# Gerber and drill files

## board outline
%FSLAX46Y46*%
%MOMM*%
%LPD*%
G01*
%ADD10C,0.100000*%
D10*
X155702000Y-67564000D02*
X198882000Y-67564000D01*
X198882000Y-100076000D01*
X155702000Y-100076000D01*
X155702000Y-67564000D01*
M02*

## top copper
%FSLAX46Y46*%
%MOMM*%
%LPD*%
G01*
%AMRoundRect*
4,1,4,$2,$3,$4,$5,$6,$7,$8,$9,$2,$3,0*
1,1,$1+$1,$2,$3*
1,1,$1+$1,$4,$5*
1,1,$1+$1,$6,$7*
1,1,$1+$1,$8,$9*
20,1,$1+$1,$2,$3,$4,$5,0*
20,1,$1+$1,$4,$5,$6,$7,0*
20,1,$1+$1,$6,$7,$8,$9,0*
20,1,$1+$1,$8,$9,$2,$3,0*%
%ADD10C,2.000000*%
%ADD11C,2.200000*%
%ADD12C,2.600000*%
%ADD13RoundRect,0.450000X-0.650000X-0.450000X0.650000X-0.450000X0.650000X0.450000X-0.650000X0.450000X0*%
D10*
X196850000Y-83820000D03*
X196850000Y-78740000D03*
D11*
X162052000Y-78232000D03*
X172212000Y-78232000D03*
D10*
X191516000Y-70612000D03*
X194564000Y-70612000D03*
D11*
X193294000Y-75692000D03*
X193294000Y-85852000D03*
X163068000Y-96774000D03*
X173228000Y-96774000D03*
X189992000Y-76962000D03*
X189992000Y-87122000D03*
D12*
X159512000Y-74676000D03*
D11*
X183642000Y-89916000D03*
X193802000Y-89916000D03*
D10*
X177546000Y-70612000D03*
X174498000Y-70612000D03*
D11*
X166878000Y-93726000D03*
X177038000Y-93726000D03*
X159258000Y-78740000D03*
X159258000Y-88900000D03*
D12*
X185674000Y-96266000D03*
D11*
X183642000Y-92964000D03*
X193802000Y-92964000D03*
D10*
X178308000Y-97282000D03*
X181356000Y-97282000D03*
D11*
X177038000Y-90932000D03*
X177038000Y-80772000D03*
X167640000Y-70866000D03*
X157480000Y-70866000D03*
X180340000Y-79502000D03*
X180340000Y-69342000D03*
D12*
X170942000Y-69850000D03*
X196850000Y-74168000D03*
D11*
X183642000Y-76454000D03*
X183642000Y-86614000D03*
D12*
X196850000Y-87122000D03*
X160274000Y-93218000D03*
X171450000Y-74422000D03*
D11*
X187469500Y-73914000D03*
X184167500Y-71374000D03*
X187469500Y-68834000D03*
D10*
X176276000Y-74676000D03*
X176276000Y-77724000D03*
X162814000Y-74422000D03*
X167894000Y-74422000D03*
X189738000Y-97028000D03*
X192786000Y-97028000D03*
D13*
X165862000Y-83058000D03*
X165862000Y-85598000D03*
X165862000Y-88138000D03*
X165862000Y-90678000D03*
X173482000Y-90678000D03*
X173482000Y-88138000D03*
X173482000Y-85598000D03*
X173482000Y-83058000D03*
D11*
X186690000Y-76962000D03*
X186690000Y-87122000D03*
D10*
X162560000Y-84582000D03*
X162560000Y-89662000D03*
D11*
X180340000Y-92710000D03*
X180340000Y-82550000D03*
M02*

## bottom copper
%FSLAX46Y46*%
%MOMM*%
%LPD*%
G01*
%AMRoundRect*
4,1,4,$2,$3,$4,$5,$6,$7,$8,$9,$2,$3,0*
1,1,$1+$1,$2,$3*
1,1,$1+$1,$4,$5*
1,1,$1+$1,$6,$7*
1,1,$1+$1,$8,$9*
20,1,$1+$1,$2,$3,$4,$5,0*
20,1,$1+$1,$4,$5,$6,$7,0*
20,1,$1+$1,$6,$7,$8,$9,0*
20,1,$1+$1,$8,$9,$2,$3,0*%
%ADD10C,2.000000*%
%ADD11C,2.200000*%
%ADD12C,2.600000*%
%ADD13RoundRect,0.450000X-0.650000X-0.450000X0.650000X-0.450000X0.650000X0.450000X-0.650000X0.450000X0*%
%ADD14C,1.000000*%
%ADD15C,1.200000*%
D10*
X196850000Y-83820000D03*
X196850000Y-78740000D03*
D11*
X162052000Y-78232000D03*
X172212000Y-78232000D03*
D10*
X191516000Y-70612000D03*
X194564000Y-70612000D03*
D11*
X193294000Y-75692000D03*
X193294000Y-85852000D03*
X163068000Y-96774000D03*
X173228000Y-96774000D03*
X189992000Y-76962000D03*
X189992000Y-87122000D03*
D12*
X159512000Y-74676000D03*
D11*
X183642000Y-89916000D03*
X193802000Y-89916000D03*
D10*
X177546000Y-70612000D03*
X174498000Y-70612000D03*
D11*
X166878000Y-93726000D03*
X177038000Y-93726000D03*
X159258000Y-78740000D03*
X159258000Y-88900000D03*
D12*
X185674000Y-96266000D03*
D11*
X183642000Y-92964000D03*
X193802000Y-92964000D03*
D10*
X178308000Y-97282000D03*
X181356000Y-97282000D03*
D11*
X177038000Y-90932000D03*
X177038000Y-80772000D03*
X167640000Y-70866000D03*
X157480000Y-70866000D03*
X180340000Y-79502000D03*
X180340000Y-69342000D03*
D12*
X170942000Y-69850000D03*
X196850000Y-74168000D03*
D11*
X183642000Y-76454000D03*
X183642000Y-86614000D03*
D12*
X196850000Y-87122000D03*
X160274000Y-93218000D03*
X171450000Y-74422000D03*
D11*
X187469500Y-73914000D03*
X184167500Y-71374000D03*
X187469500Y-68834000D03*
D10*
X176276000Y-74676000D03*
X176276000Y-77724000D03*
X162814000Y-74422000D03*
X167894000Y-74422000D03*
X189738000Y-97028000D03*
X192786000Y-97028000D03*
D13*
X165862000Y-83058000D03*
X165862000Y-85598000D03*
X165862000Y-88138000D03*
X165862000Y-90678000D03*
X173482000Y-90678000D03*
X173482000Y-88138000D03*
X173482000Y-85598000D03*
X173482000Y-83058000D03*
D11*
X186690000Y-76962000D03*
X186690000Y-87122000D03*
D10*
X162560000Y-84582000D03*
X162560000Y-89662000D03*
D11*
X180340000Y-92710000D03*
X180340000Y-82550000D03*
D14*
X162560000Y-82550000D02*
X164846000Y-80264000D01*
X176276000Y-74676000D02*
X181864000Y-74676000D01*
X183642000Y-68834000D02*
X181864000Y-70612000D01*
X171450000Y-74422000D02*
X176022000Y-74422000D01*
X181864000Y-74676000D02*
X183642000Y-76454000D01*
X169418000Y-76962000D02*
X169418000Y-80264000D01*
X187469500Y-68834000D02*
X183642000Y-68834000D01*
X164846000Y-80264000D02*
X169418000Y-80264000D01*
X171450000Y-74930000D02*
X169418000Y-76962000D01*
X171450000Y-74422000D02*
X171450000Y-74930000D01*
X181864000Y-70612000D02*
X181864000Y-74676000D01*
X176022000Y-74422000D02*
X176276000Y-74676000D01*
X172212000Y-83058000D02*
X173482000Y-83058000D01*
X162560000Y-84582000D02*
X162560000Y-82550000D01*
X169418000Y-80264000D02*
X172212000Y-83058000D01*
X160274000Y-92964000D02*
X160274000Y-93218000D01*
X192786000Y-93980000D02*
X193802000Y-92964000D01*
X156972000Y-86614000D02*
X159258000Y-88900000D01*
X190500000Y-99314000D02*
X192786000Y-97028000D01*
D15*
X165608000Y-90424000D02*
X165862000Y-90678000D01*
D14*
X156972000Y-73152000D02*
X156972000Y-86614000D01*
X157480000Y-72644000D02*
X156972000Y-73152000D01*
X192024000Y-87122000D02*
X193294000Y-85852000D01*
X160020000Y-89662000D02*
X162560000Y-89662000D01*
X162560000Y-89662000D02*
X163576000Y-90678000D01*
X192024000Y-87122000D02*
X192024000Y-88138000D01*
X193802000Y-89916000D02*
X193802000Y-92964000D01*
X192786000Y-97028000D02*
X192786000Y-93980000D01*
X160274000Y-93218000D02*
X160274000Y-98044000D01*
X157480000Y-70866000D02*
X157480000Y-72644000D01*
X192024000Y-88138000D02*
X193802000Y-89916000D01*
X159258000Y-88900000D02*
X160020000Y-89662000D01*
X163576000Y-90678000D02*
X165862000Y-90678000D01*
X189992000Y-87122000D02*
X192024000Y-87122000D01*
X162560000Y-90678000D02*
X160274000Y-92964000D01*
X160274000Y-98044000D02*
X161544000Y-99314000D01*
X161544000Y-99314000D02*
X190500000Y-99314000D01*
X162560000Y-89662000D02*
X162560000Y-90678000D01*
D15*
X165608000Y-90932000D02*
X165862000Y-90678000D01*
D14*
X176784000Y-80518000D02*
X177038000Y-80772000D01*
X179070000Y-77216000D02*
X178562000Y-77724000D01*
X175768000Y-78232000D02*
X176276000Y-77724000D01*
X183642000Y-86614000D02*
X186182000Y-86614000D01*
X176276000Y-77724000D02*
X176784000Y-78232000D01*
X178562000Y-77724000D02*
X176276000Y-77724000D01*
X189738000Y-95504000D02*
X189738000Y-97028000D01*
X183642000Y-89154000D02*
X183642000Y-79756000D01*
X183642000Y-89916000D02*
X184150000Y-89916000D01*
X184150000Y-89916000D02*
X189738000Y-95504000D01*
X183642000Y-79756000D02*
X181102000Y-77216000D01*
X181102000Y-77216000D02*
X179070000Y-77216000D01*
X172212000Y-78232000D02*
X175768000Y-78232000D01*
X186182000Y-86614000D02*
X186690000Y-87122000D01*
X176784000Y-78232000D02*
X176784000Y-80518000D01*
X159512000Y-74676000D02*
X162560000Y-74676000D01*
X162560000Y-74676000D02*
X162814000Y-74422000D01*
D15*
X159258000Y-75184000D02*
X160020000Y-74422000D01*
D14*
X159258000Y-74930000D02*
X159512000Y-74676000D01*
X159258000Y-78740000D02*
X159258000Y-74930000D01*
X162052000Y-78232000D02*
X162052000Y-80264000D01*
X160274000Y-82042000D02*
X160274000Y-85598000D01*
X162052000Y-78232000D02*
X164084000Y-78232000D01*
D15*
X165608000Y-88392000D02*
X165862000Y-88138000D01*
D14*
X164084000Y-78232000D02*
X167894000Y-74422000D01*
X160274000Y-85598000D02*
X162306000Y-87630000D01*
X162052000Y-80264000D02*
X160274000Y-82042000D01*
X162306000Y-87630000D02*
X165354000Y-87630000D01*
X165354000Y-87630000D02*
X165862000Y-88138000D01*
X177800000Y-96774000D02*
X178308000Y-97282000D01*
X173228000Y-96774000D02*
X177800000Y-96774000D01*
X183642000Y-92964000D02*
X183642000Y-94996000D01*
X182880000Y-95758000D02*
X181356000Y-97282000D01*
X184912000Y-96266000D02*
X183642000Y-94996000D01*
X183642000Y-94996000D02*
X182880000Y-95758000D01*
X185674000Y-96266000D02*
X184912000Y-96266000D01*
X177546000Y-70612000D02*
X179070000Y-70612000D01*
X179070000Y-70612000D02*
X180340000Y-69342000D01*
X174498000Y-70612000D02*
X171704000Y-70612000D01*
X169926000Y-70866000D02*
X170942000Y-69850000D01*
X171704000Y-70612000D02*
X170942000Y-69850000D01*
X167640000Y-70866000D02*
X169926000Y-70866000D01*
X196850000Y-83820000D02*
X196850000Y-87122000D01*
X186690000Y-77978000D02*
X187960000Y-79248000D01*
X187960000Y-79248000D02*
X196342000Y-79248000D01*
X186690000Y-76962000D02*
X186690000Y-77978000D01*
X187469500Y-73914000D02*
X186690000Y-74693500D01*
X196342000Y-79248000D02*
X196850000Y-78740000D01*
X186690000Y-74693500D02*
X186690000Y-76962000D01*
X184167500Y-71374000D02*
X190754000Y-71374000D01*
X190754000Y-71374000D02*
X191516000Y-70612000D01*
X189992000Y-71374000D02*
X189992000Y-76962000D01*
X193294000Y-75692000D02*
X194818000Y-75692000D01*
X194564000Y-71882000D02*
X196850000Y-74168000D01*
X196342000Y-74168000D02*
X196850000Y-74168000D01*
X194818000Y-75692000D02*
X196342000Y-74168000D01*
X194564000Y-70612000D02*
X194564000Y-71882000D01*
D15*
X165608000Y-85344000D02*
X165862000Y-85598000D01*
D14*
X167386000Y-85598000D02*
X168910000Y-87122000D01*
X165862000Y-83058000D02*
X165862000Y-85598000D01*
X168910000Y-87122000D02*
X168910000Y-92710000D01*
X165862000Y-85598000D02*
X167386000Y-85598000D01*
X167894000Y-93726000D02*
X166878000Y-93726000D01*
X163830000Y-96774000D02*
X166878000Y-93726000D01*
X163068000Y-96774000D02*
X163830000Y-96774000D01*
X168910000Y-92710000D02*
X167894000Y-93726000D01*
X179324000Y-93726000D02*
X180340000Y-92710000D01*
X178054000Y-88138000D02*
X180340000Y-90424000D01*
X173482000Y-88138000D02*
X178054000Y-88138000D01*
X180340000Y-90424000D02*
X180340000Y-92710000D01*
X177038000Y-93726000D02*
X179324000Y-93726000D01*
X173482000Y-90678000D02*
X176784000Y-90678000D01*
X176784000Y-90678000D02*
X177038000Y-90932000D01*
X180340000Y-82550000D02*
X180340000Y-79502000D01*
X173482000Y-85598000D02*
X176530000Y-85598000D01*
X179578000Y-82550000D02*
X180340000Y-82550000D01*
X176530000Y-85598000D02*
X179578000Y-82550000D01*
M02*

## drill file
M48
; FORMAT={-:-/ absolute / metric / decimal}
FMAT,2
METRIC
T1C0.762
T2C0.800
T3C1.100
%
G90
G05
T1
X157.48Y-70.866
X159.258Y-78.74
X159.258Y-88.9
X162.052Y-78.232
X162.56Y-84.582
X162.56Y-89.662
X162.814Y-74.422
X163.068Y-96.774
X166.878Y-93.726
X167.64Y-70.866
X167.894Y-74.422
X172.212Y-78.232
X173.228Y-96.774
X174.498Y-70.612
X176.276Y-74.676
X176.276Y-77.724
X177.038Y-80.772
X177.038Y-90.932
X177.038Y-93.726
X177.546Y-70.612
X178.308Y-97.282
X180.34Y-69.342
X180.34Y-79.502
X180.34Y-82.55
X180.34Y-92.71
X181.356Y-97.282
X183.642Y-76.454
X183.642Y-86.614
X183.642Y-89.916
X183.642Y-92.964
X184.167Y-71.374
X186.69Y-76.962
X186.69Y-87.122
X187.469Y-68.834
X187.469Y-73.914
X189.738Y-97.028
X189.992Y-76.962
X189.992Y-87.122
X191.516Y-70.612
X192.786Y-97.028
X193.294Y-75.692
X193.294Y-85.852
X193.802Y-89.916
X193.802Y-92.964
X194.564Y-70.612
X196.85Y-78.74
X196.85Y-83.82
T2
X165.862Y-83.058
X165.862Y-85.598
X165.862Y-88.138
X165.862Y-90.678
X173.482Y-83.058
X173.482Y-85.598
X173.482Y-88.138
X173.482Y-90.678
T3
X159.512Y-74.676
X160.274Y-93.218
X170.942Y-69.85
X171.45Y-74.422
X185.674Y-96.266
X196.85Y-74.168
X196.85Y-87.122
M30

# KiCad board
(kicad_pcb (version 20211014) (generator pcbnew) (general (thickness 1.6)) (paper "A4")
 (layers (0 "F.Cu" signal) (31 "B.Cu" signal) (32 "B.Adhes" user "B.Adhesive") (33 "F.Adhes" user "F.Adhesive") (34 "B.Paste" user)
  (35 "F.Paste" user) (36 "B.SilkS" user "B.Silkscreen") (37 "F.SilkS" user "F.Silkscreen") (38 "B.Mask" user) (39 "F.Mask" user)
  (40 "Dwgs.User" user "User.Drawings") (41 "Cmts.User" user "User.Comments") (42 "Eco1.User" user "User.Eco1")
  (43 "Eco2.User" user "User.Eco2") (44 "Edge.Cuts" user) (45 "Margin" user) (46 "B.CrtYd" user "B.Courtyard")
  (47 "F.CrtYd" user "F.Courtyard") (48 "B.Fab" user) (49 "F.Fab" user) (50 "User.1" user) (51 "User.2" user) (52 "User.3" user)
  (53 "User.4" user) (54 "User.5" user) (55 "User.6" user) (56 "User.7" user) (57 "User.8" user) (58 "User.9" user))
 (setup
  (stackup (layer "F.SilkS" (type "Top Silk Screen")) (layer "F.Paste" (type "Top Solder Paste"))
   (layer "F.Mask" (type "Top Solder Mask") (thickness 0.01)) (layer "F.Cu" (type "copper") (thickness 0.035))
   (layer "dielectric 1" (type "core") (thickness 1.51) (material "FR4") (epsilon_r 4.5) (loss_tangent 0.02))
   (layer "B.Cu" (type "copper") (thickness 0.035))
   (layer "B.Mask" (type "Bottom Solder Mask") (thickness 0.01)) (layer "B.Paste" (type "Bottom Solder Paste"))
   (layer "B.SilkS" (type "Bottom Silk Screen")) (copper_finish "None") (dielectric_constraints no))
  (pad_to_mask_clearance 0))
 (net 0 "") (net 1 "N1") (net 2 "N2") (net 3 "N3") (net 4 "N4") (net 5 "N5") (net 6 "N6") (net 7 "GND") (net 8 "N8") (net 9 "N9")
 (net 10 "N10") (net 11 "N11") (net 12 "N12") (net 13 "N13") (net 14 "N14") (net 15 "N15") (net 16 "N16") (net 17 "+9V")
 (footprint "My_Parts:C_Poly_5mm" (layer "F.Cu") (at 196.85 81.28 90)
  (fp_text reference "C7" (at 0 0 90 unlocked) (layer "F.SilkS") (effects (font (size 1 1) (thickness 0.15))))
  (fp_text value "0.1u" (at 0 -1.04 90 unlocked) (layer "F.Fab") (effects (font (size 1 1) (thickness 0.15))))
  (pad "1" thru_hole circle (at -2.54 0 90) (size 2 2) (drill 0.762) (layers *.Cu *.Mask) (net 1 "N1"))
  (pad "2" thru_hole circle (at 2.54 0 90) (size 2 2) (drill 0.762) (layers *.Cu *.Mask) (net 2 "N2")))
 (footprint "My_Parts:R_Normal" (layer "F.Cu") (at 167.132 78.232)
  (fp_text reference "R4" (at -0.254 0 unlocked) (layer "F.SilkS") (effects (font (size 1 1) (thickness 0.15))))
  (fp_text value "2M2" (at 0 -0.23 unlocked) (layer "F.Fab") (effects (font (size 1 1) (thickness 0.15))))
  (pad "1" thru_hole circle (at -5.08 0) (size 2.2 2.2) (drill 0.762) (layers *.Cu *.Mask) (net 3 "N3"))
  (pad "2" thru_hole circle (at 5.08 0) (size 2.2 2.2) (drill 0.762) (layers *.Cu *.Mask) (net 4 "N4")))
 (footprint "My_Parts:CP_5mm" (layer "F.Cu") (at 193.04 70.612)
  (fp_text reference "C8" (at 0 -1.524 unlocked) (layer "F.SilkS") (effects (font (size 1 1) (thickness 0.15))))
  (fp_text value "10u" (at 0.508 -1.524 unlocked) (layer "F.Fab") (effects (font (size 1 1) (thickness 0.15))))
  (pad "1" thru_hole circle (at -1.524 0) (size 2 2) (drill 0.762) (layers *.Cu *.Mask) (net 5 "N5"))
  (pad "2" thru_hole circle (at 1.524 0) (size 2 2) (drill 0.762) (layers *.Cu *.Mask) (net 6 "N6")))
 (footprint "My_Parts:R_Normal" (layer "F.Cu") (at 193.294 80.772 -90)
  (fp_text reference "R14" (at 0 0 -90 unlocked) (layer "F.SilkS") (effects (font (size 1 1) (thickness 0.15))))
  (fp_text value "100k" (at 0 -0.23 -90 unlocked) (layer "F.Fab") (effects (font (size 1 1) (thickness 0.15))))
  (pad "1" thru_hole circle (at -5.08 0 270) (size 2.2 2.2) (drill 0.762) (layers *.Cu *.Mask) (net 6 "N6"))
  (pad "2" thru_hole circle (at 5.08 0 270) (size 2.2 2.2) (drill 0.762) (layers *.Cu *.Mask) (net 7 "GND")))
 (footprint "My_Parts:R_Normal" (layer "F.Cu") (at 168.148 96.774)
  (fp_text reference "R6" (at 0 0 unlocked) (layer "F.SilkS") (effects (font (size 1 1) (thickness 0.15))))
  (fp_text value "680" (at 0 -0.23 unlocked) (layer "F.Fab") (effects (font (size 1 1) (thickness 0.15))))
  (pad "1" thru_hole circle (at -5.08 0) (size 2.2 2.2) (drill 0.762) (layers *.Cu *.Mask) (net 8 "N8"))
  (pad "2" thru_hole circle (at 5.08 0) (size 2.2 2.2) (drill 0.762) (layers *.Cu *.Mask) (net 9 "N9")))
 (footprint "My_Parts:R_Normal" (layer "F.Cu") (at 189.992 82.042 -90)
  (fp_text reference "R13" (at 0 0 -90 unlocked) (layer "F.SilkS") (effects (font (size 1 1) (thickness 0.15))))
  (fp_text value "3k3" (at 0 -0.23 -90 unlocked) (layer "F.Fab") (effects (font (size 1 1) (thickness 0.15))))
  (pad "1" thru_hole circle (at -5.08 0 270) (size 2.2 2.2) (drill 0.762) (layers *.Cu *.Mask) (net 5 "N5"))
  (pad "2" thru_hole circle (at 5.08 0 270) (size 2.2 2.2) (drill 0.762) (layers *.Cu *.Mask) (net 7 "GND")))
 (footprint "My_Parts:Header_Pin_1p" (layer "F.Cu") (at 159.512 74.676)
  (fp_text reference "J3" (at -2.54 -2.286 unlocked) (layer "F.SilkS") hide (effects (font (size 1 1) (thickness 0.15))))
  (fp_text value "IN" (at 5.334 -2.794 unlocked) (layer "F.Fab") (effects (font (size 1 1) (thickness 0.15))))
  (pad "1" thru_hole circle (at 0 0) (size 2.6 2.6) (drill 1.1) (layers *.Cu *.Mask) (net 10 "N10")))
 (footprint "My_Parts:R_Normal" (layer "F.Cu") (at 188.722 89.916)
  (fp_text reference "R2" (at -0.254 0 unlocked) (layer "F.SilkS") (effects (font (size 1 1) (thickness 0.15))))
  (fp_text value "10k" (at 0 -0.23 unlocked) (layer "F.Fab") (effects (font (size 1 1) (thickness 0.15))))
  (pad "1" thru_hole circle (at -5.08 0) (size 2.2 2.2) (drill 0.762) (layers *.Cu *.Mask) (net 4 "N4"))
  (pad "2" thru_hole circle (at 5.08 0) (size 2.2 2.2) (drill 0.762) (layers *.Cu *.Mask) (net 7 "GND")))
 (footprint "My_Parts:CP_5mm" (layer "F.Cu") (at 176.022 70.612 180)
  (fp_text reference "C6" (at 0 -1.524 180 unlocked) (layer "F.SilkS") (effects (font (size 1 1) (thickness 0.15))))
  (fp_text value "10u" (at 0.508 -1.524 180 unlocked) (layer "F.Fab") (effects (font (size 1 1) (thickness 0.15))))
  (pad "1" thru_hole circle (at -1.524 0 180) (size 2 2) (drill 0.762) (layers *.Cu *.Mask) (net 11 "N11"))
  (pad "2" thru_hole circle (at 1.524 0 180) (size 2 2) (drill 0.762) (layers *.Cu *.Mask) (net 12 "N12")))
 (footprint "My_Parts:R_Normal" (layer "F.Cu") (at 171.958 93.726)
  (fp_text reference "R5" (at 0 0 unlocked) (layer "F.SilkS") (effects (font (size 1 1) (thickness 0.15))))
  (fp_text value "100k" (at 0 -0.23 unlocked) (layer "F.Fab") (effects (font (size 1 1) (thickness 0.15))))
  (pad "1" thru_hole circle (at -5.08 0) (size 2.2 2.2) (drill 0.762) (layers *.Cu *.Mask) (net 8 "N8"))
  (pad "2" thru_hole circle (at 5.08 0) (size 2.2 2.2) (drill 0.762) (layers *.Cu *.Mask) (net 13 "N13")))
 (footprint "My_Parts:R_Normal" (layer "F.Cu") (at 159.258 83.82 -90)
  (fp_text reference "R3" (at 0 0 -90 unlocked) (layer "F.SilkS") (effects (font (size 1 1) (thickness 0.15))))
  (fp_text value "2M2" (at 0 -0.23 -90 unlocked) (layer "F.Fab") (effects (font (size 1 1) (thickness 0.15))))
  (pad "1" thru_hole circle (at -5.08 0 270) (size 2.2 2.2) (drill 0.762) (layers *.Cu *.Mask) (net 10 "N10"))
  (pad "2" thru_hole circle (at 5.08 0 270) (size 2.2 2.2) (drill 0.762) (layers *.Cu *.Mask) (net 7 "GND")))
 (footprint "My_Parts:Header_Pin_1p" (layer "F.Cu") (at 185.674 96.266)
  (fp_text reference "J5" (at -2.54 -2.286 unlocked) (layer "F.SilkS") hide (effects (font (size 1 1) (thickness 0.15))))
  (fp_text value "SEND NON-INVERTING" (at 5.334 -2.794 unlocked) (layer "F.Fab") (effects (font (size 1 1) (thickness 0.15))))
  (pad "1" thru_hole circle (at 0 0) (size 2.6 2.6) (drill 1.1) (layers *.Cu *.Mask) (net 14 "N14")))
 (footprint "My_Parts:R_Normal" (layer "F.Cu") (at 188.722 92.964)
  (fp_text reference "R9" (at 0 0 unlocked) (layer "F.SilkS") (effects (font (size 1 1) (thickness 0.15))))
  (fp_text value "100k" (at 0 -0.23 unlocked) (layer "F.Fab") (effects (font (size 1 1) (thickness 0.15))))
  (pad "1" thru_hole circle (at -5.08 0) (size 2.2 2.2) (drill 0.762) (layers *.Cu *.Mask) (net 14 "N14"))
  (pad "2" thru_hole circle (at 5.08 0) (size 2.2 2.2) (drill 0.762) (layers *.Cu *.Mask) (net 7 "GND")))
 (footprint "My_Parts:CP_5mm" (layer "F.Cu") (at 179.832 97.282)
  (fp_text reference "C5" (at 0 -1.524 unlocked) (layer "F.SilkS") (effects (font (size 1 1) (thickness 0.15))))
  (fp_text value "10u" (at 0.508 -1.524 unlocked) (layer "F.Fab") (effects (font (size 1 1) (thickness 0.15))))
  (pad "1" thru_hole circle (at -1.524 0) (size 2 2) (drill 0.762) (layers *.Cu *.Mask) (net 9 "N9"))
  (pad "2" thru_hole circle (at 1.524 0) (size 2 2) (drill 0.762) (layers *.Cu *.Mask) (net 14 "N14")))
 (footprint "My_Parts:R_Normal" (layer "F.Cu") (at 177.038 85.852 90)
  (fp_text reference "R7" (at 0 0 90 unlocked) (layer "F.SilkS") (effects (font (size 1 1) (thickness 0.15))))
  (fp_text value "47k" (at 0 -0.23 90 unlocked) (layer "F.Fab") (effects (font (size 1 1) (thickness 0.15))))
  (pad "1" thru_hole circle (at -5.08 0 90) (size 2.2 2.2) (drill 0.762) (layers *.Cu *.Mask) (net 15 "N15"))
  (pad "2" thru_hole circle (at 5.08 0 90) (size 2.2 2.2) (drill 0.762) (layers *.Cu *.Mask) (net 4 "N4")))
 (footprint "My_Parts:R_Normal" (layer "F.Cu") (at 162.56 70.866 180)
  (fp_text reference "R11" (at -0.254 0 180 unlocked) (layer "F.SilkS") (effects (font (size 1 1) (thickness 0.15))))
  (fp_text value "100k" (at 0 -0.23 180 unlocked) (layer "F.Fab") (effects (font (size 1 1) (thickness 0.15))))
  (pad "1" thru_hole circle (at -5.08 0 180) (size 2.2 2.2) (drill 0.762) (layers *.Cu *.Mask) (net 12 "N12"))
  (pad "2" thru_hole circle (at 5.08 0 180) (size 2.2 2.2) (drill 0.762) (layers *.Cu *.Mask) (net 7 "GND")))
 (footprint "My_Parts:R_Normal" (layer "F.Cu") (at 180.34 74.422 90)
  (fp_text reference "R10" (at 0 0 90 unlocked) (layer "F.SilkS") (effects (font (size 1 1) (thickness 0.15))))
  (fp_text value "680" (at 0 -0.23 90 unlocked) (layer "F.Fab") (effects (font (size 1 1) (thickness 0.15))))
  (pad "1" thru_hole circle (at -5.08 0 90) (size 2.2 2.2) (drill 0.762) (layers *.Cu *.Mask) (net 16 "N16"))
  (pad "2" thru_hole circle (at 5.08 0 90) (size 2.2 2.2) (drill 0.762) (layers *.Cu *.Mask) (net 11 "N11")))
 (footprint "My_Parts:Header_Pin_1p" (layer "F.Cu") (at 170.942 69.85)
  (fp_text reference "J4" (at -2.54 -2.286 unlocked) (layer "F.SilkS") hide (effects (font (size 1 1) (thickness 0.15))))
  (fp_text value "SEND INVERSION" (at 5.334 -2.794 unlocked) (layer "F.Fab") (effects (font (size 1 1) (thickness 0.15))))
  (pad "1" thru_hole circle (at 0 0) (size 2.6 2.6) (drill 1.1) (layers *.Cu *.Mask) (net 12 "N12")))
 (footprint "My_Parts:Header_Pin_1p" (layer "F.Cu") (at 196.85 74.168)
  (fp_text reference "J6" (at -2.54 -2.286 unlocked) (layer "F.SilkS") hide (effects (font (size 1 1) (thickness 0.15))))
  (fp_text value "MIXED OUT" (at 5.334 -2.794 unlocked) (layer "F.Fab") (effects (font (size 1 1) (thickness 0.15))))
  (pad "1" thru_hole circle (at 0 0) (size 2.6 2.6) (drill 1.1) (layers *.Cu *.Mask) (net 6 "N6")))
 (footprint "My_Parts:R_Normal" (layer "F.Cu") (at 183.642 81.534 -90)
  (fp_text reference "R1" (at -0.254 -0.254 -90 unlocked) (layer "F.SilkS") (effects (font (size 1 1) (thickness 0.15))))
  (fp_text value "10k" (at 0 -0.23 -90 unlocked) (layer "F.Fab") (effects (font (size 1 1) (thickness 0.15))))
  (pad "1" thru_hole circle (at -5.08 0 270) (size 2.2 2.2) (drill 0.762) (layers *.Cu *.Mask) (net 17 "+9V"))
  (pad "2" thru_hole circle (at 5.08 0 270) (size 2.2 2.2) (drill 0.762) (layers *.Cu *.Mask) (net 4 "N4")))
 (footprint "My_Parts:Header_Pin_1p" (layer "F.Cu") (at 196.85 87.122)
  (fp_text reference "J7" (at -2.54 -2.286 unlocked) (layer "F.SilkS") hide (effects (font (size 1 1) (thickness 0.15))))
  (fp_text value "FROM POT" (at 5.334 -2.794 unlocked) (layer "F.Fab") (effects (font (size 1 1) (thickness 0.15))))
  (pad "1" thru_hole circle (at 0 0) (size 2.6 2.6) (drill 1.1) (layers *.Cu *.Mask) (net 1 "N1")))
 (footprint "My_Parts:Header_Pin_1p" (layer "F.Cu") (at 160.274 93.218)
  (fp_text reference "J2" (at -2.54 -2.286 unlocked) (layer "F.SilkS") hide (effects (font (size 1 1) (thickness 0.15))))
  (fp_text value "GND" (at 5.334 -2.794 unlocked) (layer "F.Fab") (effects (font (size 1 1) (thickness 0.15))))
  (pad "1" thru_hole circle (at 0 0) (size 2.6 2.6) (drill 1.1) (layers *.Cu *.Mask) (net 7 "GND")))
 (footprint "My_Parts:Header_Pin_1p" (layer "F.Cu") (at 171.45 74.422)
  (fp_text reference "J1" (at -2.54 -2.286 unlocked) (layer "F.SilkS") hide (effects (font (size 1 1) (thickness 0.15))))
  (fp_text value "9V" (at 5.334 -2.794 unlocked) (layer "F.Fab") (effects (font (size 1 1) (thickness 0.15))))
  (pad "1" thru_hole circle (at 0 0) (size 2.6 2.6) (drill 1.1) (layers *.Cu *.Mask) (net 17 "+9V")))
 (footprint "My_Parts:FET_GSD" (layer "F.Cu") (at 186.4535 73.914 90)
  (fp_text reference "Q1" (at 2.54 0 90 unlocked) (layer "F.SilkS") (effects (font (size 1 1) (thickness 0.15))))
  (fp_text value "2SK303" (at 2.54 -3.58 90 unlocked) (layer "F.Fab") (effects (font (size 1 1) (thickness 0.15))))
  (pad "1" thru_hole circle (at 0 1.016 90) (size 2.2 2.2) (drill 0.762) (layers *.Cu *.Mask) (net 2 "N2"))
  (pad "2" thru_hole circle (at 2.54 -2.286 90) (size 2.2 2.2) (drill 0.762) (layers *.Cu *.Mask) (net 5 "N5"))
  (pad "3" thru_hole circle (at 5.08 1.016 90) (size 2.2 2.2) (drill 0.762) (layers *.Cu *.Mask) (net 17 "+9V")))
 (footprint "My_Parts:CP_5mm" (layer "F.Cu") (at 176.276 76.2 -90)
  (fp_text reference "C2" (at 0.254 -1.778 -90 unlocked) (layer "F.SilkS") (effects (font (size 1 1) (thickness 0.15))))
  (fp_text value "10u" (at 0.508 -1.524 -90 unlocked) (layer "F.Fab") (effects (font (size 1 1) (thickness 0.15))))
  (pad "1" thru_hole circle (at -1.524 0 270) (size 2 2) (drill 0.762) (layers *.Cu *.Mask) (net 17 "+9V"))
  (pad "2" thru_hole circle (at 1.524 0 270) (size 2 2) (drill 0.762) (layers *.Cu *.Mask) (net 4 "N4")))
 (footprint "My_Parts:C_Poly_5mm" (layer "F.Cu") (at 165.354 74.422)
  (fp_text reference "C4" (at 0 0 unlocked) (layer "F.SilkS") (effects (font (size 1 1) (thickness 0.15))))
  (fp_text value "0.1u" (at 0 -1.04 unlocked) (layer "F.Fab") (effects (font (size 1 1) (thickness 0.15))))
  (pad "1" thru_hole circle (at -2.54 0) (size 2 2) (drill 0.762) (layers *.Cu *.Mask) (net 10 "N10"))
  (pad "2" thru_hole circle (at 2.54 0) (size 2 2) (drill 0.762) (layers *.Cu *.Mask) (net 3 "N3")))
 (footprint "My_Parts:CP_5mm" (layer "F.Cu") (at 191.262 97.028)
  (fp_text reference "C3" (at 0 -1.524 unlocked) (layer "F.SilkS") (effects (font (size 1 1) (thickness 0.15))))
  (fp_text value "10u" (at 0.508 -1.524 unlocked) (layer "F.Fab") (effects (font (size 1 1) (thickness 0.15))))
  (pad "1" thru_hole circle (at -1.524 0) (size 2 2) (drill 0.762) (layers *.Cu *.Mask) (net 4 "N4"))
  (pad "2" thru_hole circle (at 1.524 0) (size 2 2) (drill 0.762) (layers *.Cu *.Mask) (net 7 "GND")))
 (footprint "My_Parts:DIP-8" (layer "F.Cu") (at 167.132 83.558)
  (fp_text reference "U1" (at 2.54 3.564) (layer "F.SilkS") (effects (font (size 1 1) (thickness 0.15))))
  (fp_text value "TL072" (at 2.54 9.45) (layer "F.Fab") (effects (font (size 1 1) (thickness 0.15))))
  (pad "1" thru_hole roundrect (at -1.27 -0.5) (size 2.2 1.8) (drill 0.8) (layers *.Cu *.Mask) (roundrect_rratio 0.25) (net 8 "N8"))
  (pad "2" thru_hole roundrect (at -1.27 2.04) (size 2.2 1.8) (drill 0.8) (layers *.Cu *.Mask) (roundrect_rratio 0.25) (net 8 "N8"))
  (pad "3" thru_hole roundrect (at -1.27 4.58) (size 2.2 1.8) (drill 0.8) (layers *.Cu *.Mask) (roundrect_rratio 0.25) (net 3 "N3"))
  (pad "4" thru_hole roundrect (at -1.27 7.12) (size 2.2 1.8) (drill 0.8) (layers *.Cu *.Mask) (roundrect_rratio 0.25) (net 7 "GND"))
  (pad "5" thru_hole roundrect (at 6.35 7.12) (size 2.2 1.8) (drill 0.8) (layers *.Cu *.Mask) (roundrect_rratio 0.25) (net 15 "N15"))
  (pad "6" thru_hole roundrect (at 6.35 4.58) (size 2.2 1.8) (drill 0.8) (layers *.Cu *.Mask) (roundrect_rratio 0.25) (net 13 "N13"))
  (pad "7" thru_hole roundrect (at 6.35 2.04) (size 2.2 1.8) (drill 0.8) (layers *.Cu *.Mask) (roundrect_rratio 0.25) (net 16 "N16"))
  (pad "8" thru_hole roundrect (at 6.35 -0.5) (size 2.2 1.8) (drill 0.8) (layers *.Cu *.Mask) (roundrect_rratio 0.25) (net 17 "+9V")))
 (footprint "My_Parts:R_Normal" (layer "F.Cu") (at 186.69 82.042 -90)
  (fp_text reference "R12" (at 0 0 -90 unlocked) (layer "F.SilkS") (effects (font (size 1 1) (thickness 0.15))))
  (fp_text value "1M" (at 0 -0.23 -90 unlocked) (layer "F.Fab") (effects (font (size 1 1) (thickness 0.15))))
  (pad "1" thru_hole circle (at -5.08 0 270) (size 2.2 2.2) (drill 0.762) (layers *.Cu *.Mask) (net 2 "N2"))
  (pad "2" thru_hole circle (at 5.08 0 270) (size 2.2 2.2) (drill 0.762) (layers *.Cu *.Mask) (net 4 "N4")))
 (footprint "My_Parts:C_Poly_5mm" (layer "F.Cu") (at 162.56 87.122 -90)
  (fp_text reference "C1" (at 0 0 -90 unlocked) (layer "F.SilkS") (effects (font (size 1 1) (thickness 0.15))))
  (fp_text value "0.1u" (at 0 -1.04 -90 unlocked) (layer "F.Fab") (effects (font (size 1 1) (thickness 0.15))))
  (pad "1" thru_hole circle (at -2.54 0 270) (size 2 2) (drill 0.762) (layers *.Cu *.Mask) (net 17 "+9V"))
  (pad "2" thru_hole circle (at 2.54 0 270) (size 2 2) (drill 0.762) (layers *.Cu *.Mask) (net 7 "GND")))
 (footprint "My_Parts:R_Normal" (layer "F.Cu") (at 180.34 87.63 90)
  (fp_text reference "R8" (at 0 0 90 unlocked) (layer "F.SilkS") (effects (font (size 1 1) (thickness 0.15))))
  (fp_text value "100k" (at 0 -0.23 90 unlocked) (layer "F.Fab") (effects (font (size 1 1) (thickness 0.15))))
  (pad "1" thru_hole circle (at -5.08 0 90) (size 2.2 2.2) (drill 0.762) (layers *.Cu *.Mask) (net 13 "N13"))
  (pad "2" thru_hole circle (at 5.08 0 90) (size 2.2 2.2) (drill 0.762) (layers *.Cu *.Mask) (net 16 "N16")))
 (gr_rect (start 198.882 100.076) (end 155.702 67.564) (layer "Edge.Cuts") (width 0.1) (fill none))
 (segment (start 162.56 82.55) (end 164.846 80.264) (width 1) (layer "B.Cu") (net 17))
 (segment (start 176.276 74.676) (end 181.864 74.676) (width 1) (layer "B.Cu") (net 17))
 (segment (start 183.642 68.834) (end 181.864 70.612) (width 1) (layer "B.Cu") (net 17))
 (segment (start 171.45 74.422) (end 176.022 74.422) (width 1) (layer "B.Cu") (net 17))
 (segment (start 181.864 74.676) (end 183.642 76.454) (width 1) (layer "B.Cu") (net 17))
 (segment (start 169.418 76.962) (end 169.418 80.264) (width 1) (layer "B.Cu") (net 17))
 (segment (start 187.4695 68.834) (end 183.642 68.834) (width 1) (layer "B.Cu") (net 17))
 (segment (start 164.846 80.264) (end 169.418 80.264) (width 1) (layer "B.Cu") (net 17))
 (segment (start 171.45 74.93) (end 169.418 76.962) (width 1) (layer "B.Cu") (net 17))
 (segment (start 171.45 74.422) (end 171.45 74.93) (width 1) (layer "B.Cu") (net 17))
 (segment (start 181.864 70.612) (end 181.864 74.676) (width 1) (layer "B.Cu") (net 17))
 (segment (start 176.022 74.422) (end 176.276 74.676) (width 1) (layer "B.Cu") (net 17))
 (segment (start 172.212 83.058) (end 173.482 83.058) (width 1) (layer "B.Cu") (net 17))
 (segment (start 162.56 84.582) (end 162.56 82.55) (width 1) (layer "B.Cu") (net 17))
 (segment (start 169.418 80.264) (end 172.212 83.058) (width 1) (layer "B.Cu") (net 17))
 (segment (start 160.274 92.964) (end 160.274 93.218) (width 1) (layer "B.Cu") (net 7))
 (segment (start 192.786 93.98) (end 193.802 92.964) (width 1) (layer "B.Cu") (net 7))
 (segment (start 156.972 86.614) (end 159.258 88.9) (width 1) (layer "B.Cu") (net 7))
 (segment (start 190.5 99.314) (end 192.786 97.028) (width 1) (layer "B.Cu") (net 7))
 (segment (start 165.608 90.424) (end 165.862 90.678) (width 1.2) (layer "B.Cu") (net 7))
 (segment (start 156.972 73.152) (end 156.972 86.614) (width 1) (layer "B.Cu") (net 7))
 (segment (start 157.48 72.644) (end 156.972 73.152) (width 1) (layer "B.Cu") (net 7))
 (segment (start 192.024 87.122) (end 193.294 85.852) (width 1) (layer "B.Cu") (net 7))
 (segment (start 160.02 89.662) (end 162.56 89.662) (width 1) (layer "B.Cu") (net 7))
 (segment (start 162.56 89.662) (end 163.576 90.678) (width 1) (layer "B.Cu") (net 7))
 (segment (start 192.024 87.122) (end 192.024 88.138) (width 1) (layer "B.Cu") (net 7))
 (segment (start 193.802 89.916) (end 193.802 92.964) (width 1) (layer "B.Cu") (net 7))
 (segment (start 192.786 97.028) (end 192.786 93.98) (width 1) (layer "B.Cu") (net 7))
 (segment (start 160.274 93.218) (end 160.274 98.044) (width 1) (layer "B.Cu") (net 7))
 (segment (start 157.48 70.866) (end 157.48 72.644) (width 1) (layer "B.Cu") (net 7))
 (segment (start 192.024 88.138) (end 193.802 89.916) (width 1) (layer "B.Cu") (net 7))
 (segment (start 159.258 88.9) (end 160.02 89.662) (width 1) (layer "B.Cu") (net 7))
 (segment (start 163.576 90.678) (end 165.862 90.678) (width 1) (layer "B.Cu") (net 7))
 (segment (start 189.992 87.122) (end 192.024 87.122) (width 1) (layer "B.Cu") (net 7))
 (segment (start 162.56 90.678) (end 160.274 92.964) (width 1) (layer "B.Cu") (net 7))
 (segment (start 160.274 98.044) (end 161.544 99.314) (width 1) (layer "B.Cu") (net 7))
 (segment (start 161.544 99.314) (end 190.5 99.314) (width 1) (layer "B.Cu") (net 7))
 (segment (start 162.56 89.662) (end 162.56 90.678) (width 1) (layer "B.Cu") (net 7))
 (segment (start 165.608 90.932) (end 165.862 90.678) (width 1.2) (layer "B.Cu") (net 7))
 (segment (start 176.784 80.518) (end 177.038 80.772) (width 1) (layer "B.Cu") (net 4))
 (segment (start 179.07 77.216) (end 178.562 77.724) (width 1) (layer "B.Cu") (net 4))
 (segment (start 175.768 78.232) (end 176.276 77.724) (width 1) (layer "B.Cu") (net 4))
 (segment (start 183.642 86.614) (end 186.182 86.614) (width 1) (layer "B.Cu") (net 4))
 (segment (start 176.276 77.724) (end 176.784 78.232) (width 1) (layer "B.Cu") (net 4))
 (segment (start 178.562 77.724) (end 176.276 77.724) (width 1) (layer "B.Cu") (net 4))
 (segment (start 189.738 95.504) (end 189.738 97.028) (width 1) (layer "B.Cu") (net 4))
 (segment (start 183.642 89.154) (end 183.642 79.756) (width 1) (layer "B.Cu") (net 4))
 (segment (start 183.642 89.916) (end 184.15 89.916) (width 1) (layer "B.Cu") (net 4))
 (segment (start 184.15 89.916) (end 189.738 95.504) (width 1) (layer "B.Cu") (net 4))
 (segment (start 183.642 79.756) (end 181.102 77.216) (width 1) (layer "B.Cu") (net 4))
 (segment (start 181.102 77.216) (end 179.07 77.216) (width 1) (layer "B.Cu") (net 4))
 (segment (start 172.212 78.232) (end 175.768 78.232) (width 1) (layer "B.Cu") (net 4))
 (segment (start 186.182 86.614) (end 186.69 87.122) (width 1) (layer "B.Cu") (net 4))
 (segment (start 176.784 78.232) (end 176.784 80.518) (width 1) (layer "B.Cu") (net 4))
 (segment (start 159.512 74.676) (end 162.56 74.676) (width 1) (layer "B.Cu") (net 10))
 (segment (start 162.56 74.676) (end 162.814 74.422) (width 1) (layer "B.Cu") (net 10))
 (segment (start 159.258 75.184) (end 160.02 74.422) (width 1.2) (layer "B.Cu") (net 10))
 (segment (start 159.258 74.93) (end 159.512 74.676) (width 1) (layer "B.Cu") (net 10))
 (segment (start 159.258 78.74) (end 159.258 74.93) (width 1) (layer "B.Cu") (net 10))
 (segment (start 162.052 78.232) (end 162.052 80.264) (width 1) (layer "B.Cu") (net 3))
 (segment (start 160.274 82.042) (end 160.274 85.598) (width 1) (layer "B.Cu") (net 3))
 (segment (start 162.052 78.232) (end 164.084 78.232) (width 1) (layer "B.Cu") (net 3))
 (segment (start 165.608 88.392) (end 165.862 88.138) (width 1.2) (layer "B.Cu") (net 3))
 (segment (start 164.084 78.232) (end 167.894 74.422) (width 1) (layer "B.Cu") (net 3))
 (segment (start 160.274 85.598) (end 162.306 87.63) (width 1) (layer "B.Cu") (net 3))
 (segment (start 162.052 80.264) (end 160.274 82.042) (width 1) (layer "B.Cu") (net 3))
 (segment (start 162.306 87.63) (end 165.354 87.63) (width 1) (layer "B.Cu") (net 3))
 (segment (start 165.354 87.63) (end 165.862 88.138) (width 1) (layer "B.Cu") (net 3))
 (segment (start 177.8 96.774) (end 178.308 97.282) (width 1) (layer "B.Cu") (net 9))
 (segment (start 173.228 96.774) (end 177.8 96.774) (width 1) (layer "B.Cu") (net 9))
 (segment (start 183.642 92.964) (end 183.642 94.996) (width 1) (layer "B.Cu") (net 14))
 (segment (start 182.88 95.758) (end 181.356 97.282) (width 1) (layer "B.Cu") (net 14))
 (segment (start 184.912 96.266) (end 183.642 94.996) (width 1) (layer "B.Cu") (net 14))
 (segment (start 183.642 94.996) (end 182.88 95.758) (width 1) (layer "B.Cu") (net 14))
 (segment (start 185.674 96.266) (end 184.912 96.266) (width 1) (layer "B.Cu") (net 14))
 (segment (start 177.546 70.612) (end 179.07 70.612) (width 1) (layer "B.Cu") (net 11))
 (segment (start 179.07 70.612) (end 180.34 69.342) (width 1) (layer "B.Cu") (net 11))
 (segment (start 174.498 70.612) (end 171.704 70.612) (width 1) (layer "B.Cu") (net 12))
 (segment (start 169.926 70.866) (end 170.942 69.85) (width 1) (layer "B.Cu") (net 12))
 (segment (start 171.704 70.612) (end 170.942 69.85) (width 1) (layer "B.Cu") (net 12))
 (segment (start 167.64 70.866) (end 169.926 70.866) (width 1) (layer "B.Cu") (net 12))
 (segment (start 196.85 83.82) (end 196.85 87.122) (width 1) (layer "B.Cu") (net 1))
 (segment (start 186.69 77.978) (end 187.96 79.248) (width 1) (layer "B.Cu") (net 2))
 (segment (start 187.96 79.248) (end 196.342 79.248) (width 1) (layer "B.Cu") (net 2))
 (segment (start 186.69 76.962) (end 186.69 77.978) (width 1) (layer "B.Cu") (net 2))
 (segment (start 187.4695 73.914) (end 186.69 74.6935) (width 1) (layer "B.Cu") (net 2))
 (segment (start 196.342 79.248) (end 196.85 78.74) (width 1) (layer "B.Cu") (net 2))
 (segment (start 186.69 74.6935) (end 186.69 76.962) (width 1) (layer "B.Cu") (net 2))
 (segment (start 184.1675 71.374) (end 190.754 71.374) (width 1) (layer "B.Cu") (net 5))
 (segment (start 190.754 71.374) (end 191.516 70.612) (width 1) (layer "B.Cu") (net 5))
 (segment (start 189.992 71.374) (end 189.992 76.962) (width 1) (layer "B.Cu") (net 5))
 (segment (start 193.294 75.692) (end 194.818 75.692) (width 1) (layer "B.Cu") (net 6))
 (segment (start 194.564 71.882) (end 196.85 74.168) (width 1) (layer "B.Cu") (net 6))
 (segment (start 196.342 74.168) (end 196.85 74.168) (width 1) (layer "B.Cu") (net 6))
 (segment (start 194.818 75.692) (end 196.342 74.168) (width 1) (layer "B.Cu") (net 6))
 (segment (start 194.564 70.612) (end 194.564 71.882) (width 1) (layer "B.Cu") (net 6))
 (segment (start 165.608 85.344) (end 165.862 85.598) (width 1.2) (layer "B.Cu") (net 8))
 (segment (start 167.386 85.598) (end 168.91 87.122) (width 1) (layer "B.Cu") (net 8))
 (segment (start 165.862 83.058) (end 165.862 85.598) (width 1) (layer "B.Cu") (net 8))
 (segment (start 168.91 87.122) (end 168.91 92.71) (width 1) (layer "B.Cu") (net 8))
 (segment (start 165.862 85.598) (end 167.386 85.598) (width 1) (layer "B.Cu") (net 8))
 (segment (start 167.894 93.726) (end 166.878 93.726) (width 1) (layer "B.Cu") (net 8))
 (segment (start 163.83 96.774) (end 166.878 93.726) (width 1) (layer "B.Cu") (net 8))
 (segment (start 163.068 96.774) (end 163.83 96.774) (width 1) (layer "B.Cu") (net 8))
 (segment (start 168.91 92.71) (end 167.894 93.726) (width 1) (layer "B.Cu") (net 8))
 (segment (start 179.324 93.726) (end 180.34 92.71) (width 1) (layer "B.Cu") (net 13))
 (segment (start 178.054 88.138) (end 180.34 90.424) (width 1) (layer "B.Cu") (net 13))
 (segment (start 173.482 88.138) (end 178.054 88.138) (width 1) (layer "B.Cu") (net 13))
 (segment (start 180.34 90.424) (end 180.34 92.71) (width 1) (layer "B.Cu") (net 13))
 (segment (start 177.038 93.726) (end 179.324 93.726) (width 1) (layer "B.Cu") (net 13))
 (segment (start 173.482 90.678) (end 176.784 90.678) (width 1) (layer "B.Cu") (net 15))
 (segment (start 176.784 90.678) (end 177.038 90.932) (width 1) (layer "B.Cu") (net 15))
 (segment (start 180.34 82.55) (end 180.34 79.502) (width 1) (layer "B.Cu") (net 16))
 (segment (start 173.482 85.598) (end 176.53 85.598) (width 1) (layer "B.Cu") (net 16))
 (segment (start 179.578 82.55) (end 180.34 82.55) (width 1) (layer "B.Cu") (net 16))
 (segment (start 176.53 85.598) (end 179.578 82.55) (width 1) (layer "B.Cu") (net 16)))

